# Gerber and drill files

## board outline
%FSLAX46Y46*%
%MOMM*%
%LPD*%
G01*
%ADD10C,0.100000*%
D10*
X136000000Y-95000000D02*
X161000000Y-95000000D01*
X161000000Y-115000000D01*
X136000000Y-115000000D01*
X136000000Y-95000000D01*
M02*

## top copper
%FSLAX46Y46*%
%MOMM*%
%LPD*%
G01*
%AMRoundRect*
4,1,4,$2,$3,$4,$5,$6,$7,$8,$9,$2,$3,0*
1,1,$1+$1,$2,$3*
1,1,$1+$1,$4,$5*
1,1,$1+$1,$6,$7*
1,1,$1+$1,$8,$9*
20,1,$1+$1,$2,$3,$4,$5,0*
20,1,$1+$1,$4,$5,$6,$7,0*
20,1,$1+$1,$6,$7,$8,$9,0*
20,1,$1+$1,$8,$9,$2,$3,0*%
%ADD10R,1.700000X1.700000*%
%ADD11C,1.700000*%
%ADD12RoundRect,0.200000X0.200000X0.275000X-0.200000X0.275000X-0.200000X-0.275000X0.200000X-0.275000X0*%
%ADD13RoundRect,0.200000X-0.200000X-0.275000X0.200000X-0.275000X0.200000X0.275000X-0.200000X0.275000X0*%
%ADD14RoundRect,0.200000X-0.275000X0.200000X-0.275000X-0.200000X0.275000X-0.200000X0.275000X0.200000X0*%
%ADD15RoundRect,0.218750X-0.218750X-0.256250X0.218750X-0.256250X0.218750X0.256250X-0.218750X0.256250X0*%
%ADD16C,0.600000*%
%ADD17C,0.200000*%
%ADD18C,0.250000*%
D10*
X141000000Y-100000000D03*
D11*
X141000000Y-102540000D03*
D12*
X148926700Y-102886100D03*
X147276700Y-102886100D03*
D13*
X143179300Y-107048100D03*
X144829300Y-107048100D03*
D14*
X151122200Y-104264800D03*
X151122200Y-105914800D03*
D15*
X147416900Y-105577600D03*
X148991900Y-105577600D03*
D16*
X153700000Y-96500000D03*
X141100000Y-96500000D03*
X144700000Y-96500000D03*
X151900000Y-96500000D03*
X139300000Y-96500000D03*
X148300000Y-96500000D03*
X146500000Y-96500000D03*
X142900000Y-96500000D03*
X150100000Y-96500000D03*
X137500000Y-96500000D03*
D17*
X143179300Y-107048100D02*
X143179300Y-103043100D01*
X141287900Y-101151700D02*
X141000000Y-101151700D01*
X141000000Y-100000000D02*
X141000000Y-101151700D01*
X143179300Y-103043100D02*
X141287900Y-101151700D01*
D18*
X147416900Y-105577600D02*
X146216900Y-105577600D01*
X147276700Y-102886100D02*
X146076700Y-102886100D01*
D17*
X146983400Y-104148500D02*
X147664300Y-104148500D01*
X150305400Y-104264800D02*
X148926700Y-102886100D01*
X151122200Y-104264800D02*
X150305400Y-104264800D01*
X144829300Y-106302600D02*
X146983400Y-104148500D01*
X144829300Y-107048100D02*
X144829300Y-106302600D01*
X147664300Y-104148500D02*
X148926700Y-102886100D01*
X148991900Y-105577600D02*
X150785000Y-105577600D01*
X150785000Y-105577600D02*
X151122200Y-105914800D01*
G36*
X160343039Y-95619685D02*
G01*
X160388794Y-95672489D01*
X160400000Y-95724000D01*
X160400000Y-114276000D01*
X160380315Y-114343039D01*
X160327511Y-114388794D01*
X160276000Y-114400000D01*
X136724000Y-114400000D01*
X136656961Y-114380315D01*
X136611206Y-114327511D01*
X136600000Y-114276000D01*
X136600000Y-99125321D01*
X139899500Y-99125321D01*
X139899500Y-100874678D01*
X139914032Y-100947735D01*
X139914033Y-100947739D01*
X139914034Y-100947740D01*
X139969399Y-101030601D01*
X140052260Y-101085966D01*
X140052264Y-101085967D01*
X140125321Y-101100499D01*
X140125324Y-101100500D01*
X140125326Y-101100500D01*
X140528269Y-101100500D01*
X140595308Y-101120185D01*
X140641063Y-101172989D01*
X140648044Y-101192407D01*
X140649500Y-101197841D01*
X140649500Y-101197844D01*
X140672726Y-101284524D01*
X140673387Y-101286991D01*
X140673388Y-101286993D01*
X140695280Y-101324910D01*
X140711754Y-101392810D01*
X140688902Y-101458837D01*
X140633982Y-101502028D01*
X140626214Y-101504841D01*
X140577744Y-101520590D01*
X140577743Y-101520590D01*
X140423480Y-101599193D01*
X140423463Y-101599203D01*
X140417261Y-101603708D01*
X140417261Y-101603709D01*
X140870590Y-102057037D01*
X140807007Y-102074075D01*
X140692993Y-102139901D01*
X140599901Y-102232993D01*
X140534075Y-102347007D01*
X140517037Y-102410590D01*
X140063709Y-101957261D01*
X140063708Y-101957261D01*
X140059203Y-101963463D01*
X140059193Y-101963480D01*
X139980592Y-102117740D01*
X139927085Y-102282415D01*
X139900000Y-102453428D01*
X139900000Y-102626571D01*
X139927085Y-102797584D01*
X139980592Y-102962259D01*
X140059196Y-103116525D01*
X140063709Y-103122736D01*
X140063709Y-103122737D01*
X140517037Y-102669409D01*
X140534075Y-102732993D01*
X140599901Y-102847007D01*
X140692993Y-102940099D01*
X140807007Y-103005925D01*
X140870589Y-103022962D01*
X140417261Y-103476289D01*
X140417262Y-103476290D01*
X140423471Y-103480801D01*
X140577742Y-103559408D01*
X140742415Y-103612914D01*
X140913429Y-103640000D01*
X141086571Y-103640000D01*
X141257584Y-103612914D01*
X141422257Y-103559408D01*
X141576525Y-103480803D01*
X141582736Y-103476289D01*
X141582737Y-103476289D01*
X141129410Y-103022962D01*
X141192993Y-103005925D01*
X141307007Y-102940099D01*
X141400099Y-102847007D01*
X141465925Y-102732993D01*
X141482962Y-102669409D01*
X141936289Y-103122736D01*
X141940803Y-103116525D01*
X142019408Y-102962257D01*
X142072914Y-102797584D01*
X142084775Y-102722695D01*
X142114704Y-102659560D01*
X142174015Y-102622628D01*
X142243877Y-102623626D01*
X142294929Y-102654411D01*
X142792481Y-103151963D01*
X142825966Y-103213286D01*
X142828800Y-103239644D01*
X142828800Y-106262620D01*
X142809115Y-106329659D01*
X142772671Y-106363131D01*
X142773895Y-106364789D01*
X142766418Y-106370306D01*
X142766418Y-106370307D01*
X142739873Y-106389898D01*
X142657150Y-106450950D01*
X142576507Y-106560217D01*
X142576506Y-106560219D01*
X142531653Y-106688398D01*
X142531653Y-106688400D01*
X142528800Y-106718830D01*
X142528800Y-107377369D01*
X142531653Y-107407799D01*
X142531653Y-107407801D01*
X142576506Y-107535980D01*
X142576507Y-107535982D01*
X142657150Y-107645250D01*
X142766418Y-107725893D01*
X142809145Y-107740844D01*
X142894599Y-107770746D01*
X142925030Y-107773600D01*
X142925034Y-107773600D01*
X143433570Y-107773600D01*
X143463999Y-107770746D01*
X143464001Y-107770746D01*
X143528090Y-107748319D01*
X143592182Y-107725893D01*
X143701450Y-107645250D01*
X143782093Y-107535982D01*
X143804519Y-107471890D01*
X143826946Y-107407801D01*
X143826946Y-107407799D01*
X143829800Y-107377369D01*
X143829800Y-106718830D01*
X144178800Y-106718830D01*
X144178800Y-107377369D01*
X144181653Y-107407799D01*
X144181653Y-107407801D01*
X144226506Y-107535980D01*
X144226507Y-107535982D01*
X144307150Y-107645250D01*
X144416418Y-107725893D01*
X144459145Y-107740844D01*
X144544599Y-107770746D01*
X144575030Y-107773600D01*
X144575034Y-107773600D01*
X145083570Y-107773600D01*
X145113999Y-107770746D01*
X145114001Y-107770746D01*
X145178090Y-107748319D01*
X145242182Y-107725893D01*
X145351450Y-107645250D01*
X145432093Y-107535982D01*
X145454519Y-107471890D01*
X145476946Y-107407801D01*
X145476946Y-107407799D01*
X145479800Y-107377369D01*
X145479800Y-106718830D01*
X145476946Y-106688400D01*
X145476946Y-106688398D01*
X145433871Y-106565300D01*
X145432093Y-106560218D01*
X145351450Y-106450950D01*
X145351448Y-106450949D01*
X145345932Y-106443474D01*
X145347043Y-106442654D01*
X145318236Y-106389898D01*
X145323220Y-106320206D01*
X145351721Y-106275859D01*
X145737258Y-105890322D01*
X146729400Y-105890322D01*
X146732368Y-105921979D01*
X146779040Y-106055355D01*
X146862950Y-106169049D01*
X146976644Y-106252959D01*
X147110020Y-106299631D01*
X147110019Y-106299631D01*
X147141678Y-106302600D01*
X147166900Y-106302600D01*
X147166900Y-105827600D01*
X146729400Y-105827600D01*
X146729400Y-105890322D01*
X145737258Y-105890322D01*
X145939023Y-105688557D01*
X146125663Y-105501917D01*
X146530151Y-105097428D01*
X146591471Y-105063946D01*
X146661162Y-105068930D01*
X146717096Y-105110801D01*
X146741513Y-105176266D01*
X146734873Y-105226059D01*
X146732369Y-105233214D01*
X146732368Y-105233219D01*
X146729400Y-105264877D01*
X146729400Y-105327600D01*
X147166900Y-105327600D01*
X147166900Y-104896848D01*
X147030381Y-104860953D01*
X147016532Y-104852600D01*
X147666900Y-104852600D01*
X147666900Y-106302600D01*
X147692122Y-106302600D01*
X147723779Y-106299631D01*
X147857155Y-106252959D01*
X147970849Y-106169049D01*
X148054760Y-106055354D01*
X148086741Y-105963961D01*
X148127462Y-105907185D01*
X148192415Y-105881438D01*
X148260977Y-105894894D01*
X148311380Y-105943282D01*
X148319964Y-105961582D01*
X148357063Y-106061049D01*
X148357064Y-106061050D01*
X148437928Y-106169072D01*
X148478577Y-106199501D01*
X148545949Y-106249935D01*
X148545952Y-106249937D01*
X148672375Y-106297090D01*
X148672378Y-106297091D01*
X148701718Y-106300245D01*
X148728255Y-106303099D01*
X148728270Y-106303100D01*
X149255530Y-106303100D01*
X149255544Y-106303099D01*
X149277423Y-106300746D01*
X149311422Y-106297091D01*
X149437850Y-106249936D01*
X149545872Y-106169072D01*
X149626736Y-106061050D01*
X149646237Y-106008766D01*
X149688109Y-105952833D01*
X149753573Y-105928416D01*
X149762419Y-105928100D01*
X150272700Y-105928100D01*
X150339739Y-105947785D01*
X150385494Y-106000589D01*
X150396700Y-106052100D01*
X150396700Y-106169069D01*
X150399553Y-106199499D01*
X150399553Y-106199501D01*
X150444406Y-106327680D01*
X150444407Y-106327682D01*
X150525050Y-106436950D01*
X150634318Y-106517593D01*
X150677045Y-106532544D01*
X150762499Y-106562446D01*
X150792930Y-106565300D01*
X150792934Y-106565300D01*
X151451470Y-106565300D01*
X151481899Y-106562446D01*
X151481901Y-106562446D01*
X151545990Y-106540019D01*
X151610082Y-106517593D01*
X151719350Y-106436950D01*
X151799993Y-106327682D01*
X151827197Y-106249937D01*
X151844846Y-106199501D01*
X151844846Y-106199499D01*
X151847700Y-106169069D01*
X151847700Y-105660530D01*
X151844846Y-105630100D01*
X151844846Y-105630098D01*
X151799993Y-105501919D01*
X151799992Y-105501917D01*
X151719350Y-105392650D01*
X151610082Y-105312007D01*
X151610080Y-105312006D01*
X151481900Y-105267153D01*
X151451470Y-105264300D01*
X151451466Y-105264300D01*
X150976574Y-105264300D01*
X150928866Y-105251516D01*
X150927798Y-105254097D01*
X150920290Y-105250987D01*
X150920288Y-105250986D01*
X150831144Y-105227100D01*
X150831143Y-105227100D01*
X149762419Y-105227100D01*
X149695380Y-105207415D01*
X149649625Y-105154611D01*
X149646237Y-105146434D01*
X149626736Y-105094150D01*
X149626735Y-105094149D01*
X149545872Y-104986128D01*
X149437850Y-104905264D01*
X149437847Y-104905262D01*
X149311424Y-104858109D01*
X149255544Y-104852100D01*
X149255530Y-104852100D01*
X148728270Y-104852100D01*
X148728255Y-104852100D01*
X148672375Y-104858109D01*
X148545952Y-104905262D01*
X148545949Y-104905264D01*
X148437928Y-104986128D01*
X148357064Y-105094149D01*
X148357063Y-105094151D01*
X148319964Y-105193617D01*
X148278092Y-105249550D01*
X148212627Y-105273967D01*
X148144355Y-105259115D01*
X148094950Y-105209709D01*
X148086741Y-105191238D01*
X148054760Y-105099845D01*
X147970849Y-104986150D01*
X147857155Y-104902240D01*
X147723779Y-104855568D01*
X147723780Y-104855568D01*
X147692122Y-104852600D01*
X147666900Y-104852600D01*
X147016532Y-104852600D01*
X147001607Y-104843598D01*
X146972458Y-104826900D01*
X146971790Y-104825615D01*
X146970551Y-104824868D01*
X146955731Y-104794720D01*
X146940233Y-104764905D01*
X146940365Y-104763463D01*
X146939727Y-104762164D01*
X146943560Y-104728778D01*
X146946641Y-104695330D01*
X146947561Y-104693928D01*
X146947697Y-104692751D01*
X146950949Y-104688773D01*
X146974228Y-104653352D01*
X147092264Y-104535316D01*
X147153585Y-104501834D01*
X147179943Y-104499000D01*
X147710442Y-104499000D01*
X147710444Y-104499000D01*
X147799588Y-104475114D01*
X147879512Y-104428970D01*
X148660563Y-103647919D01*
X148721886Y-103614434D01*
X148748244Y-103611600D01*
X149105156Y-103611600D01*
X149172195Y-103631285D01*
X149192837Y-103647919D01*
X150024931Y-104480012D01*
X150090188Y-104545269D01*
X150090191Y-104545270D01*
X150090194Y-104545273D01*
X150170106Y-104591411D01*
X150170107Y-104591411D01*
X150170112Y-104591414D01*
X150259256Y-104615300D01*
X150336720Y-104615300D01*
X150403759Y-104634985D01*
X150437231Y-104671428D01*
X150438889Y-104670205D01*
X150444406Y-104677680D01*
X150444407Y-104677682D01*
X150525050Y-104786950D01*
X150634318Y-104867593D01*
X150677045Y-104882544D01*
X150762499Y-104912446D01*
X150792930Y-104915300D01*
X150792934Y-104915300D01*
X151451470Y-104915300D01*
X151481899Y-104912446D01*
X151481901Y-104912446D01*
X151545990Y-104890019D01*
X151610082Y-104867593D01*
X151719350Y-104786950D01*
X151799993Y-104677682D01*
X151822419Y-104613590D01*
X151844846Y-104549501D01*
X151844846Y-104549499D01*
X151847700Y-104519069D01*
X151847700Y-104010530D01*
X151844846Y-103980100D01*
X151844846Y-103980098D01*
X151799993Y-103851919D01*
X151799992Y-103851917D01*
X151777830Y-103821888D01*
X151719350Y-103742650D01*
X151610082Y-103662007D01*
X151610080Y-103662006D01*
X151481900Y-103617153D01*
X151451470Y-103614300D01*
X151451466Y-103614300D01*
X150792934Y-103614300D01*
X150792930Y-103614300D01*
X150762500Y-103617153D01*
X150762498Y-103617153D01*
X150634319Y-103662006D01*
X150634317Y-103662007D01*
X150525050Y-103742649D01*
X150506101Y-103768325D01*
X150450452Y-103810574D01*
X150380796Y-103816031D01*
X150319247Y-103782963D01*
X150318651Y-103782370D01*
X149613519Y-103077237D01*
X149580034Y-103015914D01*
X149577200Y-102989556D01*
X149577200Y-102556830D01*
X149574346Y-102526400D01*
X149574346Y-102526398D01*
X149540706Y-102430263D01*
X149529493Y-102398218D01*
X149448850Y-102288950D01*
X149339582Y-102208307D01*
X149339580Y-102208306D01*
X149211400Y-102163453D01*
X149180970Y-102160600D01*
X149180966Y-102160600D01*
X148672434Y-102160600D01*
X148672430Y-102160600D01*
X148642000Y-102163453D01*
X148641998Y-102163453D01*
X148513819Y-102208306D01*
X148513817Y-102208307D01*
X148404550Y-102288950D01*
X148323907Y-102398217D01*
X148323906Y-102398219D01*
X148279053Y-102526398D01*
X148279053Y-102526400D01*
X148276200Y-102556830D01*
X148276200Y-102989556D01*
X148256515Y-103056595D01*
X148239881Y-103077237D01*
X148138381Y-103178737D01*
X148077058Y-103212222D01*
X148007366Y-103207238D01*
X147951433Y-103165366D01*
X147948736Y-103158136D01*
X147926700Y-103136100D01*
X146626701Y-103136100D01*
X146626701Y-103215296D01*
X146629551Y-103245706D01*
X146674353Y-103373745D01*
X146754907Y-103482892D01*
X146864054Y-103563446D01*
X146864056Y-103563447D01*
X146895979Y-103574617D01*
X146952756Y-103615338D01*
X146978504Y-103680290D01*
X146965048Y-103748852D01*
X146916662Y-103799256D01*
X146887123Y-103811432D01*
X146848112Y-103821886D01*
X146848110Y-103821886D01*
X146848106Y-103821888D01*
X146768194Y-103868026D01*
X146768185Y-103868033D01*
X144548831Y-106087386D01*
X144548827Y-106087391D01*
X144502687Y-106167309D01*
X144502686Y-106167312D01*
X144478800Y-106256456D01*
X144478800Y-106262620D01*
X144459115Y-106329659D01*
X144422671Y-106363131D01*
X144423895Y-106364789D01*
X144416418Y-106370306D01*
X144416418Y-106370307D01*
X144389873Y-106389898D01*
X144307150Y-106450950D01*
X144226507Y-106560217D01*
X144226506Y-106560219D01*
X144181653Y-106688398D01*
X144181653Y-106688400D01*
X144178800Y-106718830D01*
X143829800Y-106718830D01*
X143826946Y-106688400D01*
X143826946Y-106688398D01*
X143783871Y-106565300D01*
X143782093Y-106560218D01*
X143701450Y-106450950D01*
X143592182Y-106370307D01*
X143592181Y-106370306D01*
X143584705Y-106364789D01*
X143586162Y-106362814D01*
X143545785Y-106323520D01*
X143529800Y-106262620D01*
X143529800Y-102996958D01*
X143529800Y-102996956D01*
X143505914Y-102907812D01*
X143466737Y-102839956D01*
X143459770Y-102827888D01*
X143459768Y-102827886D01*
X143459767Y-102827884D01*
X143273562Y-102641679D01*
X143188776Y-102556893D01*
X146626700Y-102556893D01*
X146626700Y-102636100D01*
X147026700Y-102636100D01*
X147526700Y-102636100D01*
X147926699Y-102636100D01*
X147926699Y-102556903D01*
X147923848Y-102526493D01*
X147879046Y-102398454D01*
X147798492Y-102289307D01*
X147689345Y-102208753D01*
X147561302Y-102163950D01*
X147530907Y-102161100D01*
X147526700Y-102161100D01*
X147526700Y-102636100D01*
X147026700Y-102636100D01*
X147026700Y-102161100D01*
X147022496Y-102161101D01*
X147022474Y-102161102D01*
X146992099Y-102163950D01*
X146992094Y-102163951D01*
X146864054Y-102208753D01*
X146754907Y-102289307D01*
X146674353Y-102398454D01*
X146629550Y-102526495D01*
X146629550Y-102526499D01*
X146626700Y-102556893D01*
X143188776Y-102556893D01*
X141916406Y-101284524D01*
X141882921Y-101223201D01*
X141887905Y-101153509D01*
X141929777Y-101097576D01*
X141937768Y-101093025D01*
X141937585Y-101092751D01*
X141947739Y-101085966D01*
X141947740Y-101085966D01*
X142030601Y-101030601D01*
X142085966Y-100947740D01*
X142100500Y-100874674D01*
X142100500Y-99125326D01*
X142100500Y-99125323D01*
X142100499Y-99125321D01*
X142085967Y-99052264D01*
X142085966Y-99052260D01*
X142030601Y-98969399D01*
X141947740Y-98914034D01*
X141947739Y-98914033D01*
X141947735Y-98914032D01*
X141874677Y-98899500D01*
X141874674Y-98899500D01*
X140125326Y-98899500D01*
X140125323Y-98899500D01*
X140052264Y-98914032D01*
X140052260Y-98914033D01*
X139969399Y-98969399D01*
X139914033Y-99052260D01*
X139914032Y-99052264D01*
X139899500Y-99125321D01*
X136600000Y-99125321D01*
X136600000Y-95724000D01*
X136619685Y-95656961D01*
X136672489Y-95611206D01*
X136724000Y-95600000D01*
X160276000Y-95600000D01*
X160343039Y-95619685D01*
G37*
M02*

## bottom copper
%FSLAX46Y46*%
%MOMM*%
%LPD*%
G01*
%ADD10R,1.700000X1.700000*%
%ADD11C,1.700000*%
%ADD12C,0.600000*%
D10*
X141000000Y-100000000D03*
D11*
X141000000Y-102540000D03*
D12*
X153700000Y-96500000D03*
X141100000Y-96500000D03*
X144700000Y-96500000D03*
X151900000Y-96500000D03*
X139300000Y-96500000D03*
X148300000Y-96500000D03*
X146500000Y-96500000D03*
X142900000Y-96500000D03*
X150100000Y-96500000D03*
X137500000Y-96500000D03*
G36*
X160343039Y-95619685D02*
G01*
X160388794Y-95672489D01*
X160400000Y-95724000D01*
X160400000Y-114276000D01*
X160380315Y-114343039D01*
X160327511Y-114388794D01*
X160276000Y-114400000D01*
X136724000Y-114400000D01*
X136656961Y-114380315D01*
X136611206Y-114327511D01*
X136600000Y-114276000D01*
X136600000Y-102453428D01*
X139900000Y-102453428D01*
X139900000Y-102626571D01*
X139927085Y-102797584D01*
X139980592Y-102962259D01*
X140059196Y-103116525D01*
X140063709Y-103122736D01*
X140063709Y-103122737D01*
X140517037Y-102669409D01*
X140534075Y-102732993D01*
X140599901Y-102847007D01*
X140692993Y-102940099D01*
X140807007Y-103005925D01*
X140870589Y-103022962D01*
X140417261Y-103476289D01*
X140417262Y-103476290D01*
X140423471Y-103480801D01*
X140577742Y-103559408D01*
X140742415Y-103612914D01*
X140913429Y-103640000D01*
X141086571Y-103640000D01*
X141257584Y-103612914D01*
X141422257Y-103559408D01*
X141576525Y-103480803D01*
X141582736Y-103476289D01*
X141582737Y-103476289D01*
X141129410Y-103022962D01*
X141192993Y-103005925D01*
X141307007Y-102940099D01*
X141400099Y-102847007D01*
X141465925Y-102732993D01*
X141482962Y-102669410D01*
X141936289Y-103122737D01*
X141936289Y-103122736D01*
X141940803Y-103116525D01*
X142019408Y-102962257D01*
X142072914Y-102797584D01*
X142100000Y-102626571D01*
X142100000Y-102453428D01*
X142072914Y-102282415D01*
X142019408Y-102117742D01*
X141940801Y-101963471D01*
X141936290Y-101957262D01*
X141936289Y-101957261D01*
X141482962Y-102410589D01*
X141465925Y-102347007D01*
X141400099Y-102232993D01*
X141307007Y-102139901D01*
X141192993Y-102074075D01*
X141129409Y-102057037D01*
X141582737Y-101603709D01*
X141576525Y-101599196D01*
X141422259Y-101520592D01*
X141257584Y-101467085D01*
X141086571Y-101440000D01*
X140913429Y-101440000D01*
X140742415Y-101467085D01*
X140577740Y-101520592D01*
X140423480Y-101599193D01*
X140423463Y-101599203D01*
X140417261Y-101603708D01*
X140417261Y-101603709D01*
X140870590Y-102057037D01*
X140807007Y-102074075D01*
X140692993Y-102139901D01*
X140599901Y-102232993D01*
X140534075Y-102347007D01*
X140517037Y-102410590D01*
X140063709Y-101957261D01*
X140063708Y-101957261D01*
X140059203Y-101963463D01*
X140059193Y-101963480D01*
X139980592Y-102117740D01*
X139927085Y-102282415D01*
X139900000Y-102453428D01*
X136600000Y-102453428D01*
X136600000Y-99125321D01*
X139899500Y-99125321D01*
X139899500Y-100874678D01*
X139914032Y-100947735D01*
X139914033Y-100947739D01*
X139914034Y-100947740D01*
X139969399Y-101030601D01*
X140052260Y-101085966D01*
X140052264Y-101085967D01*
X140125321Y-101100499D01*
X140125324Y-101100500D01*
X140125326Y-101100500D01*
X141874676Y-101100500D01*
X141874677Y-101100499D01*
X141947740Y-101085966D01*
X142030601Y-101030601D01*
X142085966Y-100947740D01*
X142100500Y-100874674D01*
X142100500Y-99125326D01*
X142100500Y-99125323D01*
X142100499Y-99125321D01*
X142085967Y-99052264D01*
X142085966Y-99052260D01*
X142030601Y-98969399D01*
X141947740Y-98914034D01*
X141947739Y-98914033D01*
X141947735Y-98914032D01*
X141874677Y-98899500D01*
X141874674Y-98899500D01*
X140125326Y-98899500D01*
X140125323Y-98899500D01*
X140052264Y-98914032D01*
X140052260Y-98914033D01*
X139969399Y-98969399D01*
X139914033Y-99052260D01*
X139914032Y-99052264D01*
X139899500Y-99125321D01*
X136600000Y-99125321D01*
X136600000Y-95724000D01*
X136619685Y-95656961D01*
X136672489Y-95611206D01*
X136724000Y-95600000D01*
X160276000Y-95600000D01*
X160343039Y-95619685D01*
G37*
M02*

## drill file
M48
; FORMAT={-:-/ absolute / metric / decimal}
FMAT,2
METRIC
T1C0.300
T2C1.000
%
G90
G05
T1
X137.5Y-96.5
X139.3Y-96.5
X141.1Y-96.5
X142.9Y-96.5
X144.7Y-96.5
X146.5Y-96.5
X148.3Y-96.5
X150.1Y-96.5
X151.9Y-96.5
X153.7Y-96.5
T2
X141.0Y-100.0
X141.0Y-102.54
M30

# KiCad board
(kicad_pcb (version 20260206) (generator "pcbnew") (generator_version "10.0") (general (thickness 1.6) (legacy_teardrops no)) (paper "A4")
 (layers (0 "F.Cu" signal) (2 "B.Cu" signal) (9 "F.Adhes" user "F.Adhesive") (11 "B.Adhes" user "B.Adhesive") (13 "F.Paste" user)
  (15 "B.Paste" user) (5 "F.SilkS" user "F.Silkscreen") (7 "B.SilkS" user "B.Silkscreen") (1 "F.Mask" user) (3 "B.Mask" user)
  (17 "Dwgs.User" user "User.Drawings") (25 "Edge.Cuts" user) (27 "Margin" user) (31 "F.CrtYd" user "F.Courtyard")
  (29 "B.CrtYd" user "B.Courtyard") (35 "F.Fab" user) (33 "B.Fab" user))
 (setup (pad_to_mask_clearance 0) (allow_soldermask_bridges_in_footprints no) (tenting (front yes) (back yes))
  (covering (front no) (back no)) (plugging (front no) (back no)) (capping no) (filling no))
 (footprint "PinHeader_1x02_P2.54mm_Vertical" (layer "F.Cu") (at 141 100)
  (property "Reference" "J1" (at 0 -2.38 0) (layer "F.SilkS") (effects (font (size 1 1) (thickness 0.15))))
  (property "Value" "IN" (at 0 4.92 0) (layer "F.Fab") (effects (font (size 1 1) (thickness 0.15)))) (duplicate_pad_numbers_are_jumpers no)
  (pad "1" thru_hole rect (at 0 0) (size 1.7 1.7) (drill 1) (layers "*.Cu" "*.Mask") (remove_unused_layers no) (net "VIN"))
  (pad "2" thru_hole circle (at 0 2.54) (size 1.7 1.7) (drill 1) (layers "*.Cu" "*.Mask") (remove_unused_layers no) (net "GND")))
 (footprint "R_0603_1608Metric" (layer "F.Cu") (at 148.1017 102.8861 180)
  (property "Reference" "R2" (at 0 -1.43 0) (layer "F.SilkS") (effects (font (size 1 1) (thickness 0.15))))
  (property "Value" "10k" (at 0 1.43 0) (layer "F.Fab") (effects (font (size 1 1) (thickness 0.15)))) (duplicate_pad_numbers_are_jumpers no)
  (pad "1" smd roundrect (at -0.825 0 180) (size 0.8 0.95) (layers "F.Cu" "F.Mask" "F.Paste") (roundrect_rratio 0.25) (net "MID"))
  (pad "2" smd roundrect (at 0.825 0 180) (size 0.8 0.95) (layers "F.Cu" "F.Mask" "F.Paste") (roundrect_rratio 0.25) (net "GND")))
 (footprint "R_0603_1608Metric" (layer "F.Cu") (at 144.0043 107.0481)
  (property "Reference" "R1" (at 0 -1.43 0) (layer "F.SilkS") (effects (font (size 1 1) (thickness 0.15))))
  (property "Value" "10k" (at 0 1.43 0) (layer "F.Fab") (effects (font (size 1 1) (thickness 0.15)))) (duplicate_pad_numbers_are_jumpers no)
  (pad "1" smd roundrect (at -0.825 0) (size 0.8 0.95) (layers "F.Cu" "F.Mask" "F.Paste") (roundrect_rratio 0.25) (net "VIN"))
  (pad "2" smd roundrect (at 0.825 0) (size 0.8 0.95) (layers "F.Cu" "F.Mask" "F.Paste") (roundrect_rratio 0.25) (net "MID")))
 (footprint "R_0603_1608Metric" (layer "F.Cu") (at 151.1222 105.0898 -90)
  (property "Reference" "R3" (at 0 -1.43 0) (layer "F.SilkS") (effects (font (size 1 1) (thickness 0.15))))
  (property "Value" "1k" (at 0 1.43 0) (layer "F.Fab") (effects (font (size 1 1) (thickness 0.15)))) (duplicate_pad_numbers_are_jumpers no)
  (pad "1" smd roundrect (at -0.825 0 270) (size 0.8 0.95) (layers "F.Cu" "F.Mask" "F.Paste") (roundrect_rratio 0.25) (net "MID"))
  (pad "2" smd roundrect (at 0.825 0 270) (size 0.8 0.95) (layers "F.Cu" "F.Mask" "F.Paste") (roundrect_rratio 0.25) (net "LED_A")))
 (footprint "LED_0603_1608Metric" (layer "F.Cu") (at 148.2044 105.5776)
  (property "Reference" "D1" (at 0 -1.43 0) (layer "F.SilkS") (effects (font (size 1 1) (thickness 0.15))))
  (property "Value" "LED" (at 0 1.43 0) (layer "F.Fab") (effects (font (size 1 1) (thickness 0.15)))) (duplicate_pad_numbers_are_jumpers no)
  (pad "1" smd roundrect (at -0.7875 0) (size 0.875 0.95) (layers "F.Cu" "F.Mask" "F.Paste") (roundrect_rratio 0.25) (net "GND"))
  (pad "2" smd roundrect (at 0.7875 0) (size 0.875 0.95) (layers "F.Cu" "F.Mask" "F.Paste") (roundrect_rratio 0.25) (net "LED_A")))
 (gr_rect (start 136 95) (end 161 115) (stroke (width 0.1) (type default)) (fill no) (layer "Edge.Cuts"))
 (segment (start 143.1793 107.0481) (end 143.1793 103.0431) (width 0.2) (layer "F.Cu") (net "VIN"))
 (segment (start 141.2879 101.1517) (end 141 101.1517) (width 0.2) (layer "F.Cu") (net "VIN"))
 (segment (start 141 100) (end 141 101.1517) (width 0.2) (layer "F.Cu") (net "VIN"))
 (segment (start 143.1793 103.0431) (end 141.2879 101.1517) (width 0.2) (layer "F.Cu") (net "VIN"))
 (segment (start 147.4169 105.5776) (end 146.2169 105.5776) (width 0.25) (layer "F.Cu") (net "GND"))
 (segment (start 147.2767 102.8861) (end 146.0767 102.8861) (width 0.25) (layer "F.Cu") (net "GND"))
 (via (at 153.7 96.5) (size 0.6) (drill 0.3) (layers "F.Cu" "B.Cu") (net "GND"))
 (via (at 141.1 96.5) (size 0.6) (drill 0.3) (layers "F.Cu" "B.Cu") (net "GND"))
 (via (at 144.7 96.5) (size 0.6) (drill 0.3) (layers "F.Cu" "B.Cu") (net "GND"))
 (via (at 151.9 96.5) (size 0.6) (drill 0.3) (layers "F.Cu" "B.Cu") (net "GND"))
 (via (at 139.3 96.5) (size 0.6) (drill 0.3) (layers "F.Cu" "B.Cu") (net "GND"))
 (via (at 148.3 96.5) (size 0.6) (drill 0.3) (layers "F.Cu" "B.Cu") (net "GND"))
 (via (at 146.5 96.5) (size 0.6) (drill 0.3) (layers "F.Cu" "B.Cu") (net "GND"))
 (via (at 142.9 96.5) (size 0.6) (drill 0.3) (layers "F.Cu" "B.Cu") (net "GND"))
 (via (at 150.1 96.5) (size 0.6) (drill 0.3) (layers "F.Cu" "B.Cu") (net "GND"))
 (via (at 137.5 96.5) (size 0.6) (drill 0.3) (layers "F.Cu" "B.Cu") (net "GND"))
 (segment (start 146.9834 104.1485) (end 147.6643 104.1485) (width 0.2) (layer "F.Cu") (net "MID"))
 (segment (start 150.3054 104.2648) (end 148.9267 102.8861) (width 0.2) (layer "F.Cu") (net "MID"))
 (segment (start 151.1222 104.2648) (end 150.3054 104.2648) (width 0.2) (layer "F.Cu") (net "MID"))
 (segment (start 144.8293 106.3026) (end 146.9834 104.1485) (width 0.2) (layer "F.Cu") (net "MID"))
 (segment (start 144.8293 107.0481) (end 144.8293 106.3026) (width 0.2) (layer "F.Cu") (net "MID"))
 (segment (start 147.6643 104.1485) (end 148.9267 102.8861) (width 0.2) (layer "F.Cu") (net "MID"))
 (segment (start 148.9919 105.5776) (end 150.785 105.5776) (width 0.2) (layer "F.Cu") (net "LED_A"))
 (segment (start 150.785 105.5776) (end 151.1222 105.9148) (width 0.2) (layer "F.Cu") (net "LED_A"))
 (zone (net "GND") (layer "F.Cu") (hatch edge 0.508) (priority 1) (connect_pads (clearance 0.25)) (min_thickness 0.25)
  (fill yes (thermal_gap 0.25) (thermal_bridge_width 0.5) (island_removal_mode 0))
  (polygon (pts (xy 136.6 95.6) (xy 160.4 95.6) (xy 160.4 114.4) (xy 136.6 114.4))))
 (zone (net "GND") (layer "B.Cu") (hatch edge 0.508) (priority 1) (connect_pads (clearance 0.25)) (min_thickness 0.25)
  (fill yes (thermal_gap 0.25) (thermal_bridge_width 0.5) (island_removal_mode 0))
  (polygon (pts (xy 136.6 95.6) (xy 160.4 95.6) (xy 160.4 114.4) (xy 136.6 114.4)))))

